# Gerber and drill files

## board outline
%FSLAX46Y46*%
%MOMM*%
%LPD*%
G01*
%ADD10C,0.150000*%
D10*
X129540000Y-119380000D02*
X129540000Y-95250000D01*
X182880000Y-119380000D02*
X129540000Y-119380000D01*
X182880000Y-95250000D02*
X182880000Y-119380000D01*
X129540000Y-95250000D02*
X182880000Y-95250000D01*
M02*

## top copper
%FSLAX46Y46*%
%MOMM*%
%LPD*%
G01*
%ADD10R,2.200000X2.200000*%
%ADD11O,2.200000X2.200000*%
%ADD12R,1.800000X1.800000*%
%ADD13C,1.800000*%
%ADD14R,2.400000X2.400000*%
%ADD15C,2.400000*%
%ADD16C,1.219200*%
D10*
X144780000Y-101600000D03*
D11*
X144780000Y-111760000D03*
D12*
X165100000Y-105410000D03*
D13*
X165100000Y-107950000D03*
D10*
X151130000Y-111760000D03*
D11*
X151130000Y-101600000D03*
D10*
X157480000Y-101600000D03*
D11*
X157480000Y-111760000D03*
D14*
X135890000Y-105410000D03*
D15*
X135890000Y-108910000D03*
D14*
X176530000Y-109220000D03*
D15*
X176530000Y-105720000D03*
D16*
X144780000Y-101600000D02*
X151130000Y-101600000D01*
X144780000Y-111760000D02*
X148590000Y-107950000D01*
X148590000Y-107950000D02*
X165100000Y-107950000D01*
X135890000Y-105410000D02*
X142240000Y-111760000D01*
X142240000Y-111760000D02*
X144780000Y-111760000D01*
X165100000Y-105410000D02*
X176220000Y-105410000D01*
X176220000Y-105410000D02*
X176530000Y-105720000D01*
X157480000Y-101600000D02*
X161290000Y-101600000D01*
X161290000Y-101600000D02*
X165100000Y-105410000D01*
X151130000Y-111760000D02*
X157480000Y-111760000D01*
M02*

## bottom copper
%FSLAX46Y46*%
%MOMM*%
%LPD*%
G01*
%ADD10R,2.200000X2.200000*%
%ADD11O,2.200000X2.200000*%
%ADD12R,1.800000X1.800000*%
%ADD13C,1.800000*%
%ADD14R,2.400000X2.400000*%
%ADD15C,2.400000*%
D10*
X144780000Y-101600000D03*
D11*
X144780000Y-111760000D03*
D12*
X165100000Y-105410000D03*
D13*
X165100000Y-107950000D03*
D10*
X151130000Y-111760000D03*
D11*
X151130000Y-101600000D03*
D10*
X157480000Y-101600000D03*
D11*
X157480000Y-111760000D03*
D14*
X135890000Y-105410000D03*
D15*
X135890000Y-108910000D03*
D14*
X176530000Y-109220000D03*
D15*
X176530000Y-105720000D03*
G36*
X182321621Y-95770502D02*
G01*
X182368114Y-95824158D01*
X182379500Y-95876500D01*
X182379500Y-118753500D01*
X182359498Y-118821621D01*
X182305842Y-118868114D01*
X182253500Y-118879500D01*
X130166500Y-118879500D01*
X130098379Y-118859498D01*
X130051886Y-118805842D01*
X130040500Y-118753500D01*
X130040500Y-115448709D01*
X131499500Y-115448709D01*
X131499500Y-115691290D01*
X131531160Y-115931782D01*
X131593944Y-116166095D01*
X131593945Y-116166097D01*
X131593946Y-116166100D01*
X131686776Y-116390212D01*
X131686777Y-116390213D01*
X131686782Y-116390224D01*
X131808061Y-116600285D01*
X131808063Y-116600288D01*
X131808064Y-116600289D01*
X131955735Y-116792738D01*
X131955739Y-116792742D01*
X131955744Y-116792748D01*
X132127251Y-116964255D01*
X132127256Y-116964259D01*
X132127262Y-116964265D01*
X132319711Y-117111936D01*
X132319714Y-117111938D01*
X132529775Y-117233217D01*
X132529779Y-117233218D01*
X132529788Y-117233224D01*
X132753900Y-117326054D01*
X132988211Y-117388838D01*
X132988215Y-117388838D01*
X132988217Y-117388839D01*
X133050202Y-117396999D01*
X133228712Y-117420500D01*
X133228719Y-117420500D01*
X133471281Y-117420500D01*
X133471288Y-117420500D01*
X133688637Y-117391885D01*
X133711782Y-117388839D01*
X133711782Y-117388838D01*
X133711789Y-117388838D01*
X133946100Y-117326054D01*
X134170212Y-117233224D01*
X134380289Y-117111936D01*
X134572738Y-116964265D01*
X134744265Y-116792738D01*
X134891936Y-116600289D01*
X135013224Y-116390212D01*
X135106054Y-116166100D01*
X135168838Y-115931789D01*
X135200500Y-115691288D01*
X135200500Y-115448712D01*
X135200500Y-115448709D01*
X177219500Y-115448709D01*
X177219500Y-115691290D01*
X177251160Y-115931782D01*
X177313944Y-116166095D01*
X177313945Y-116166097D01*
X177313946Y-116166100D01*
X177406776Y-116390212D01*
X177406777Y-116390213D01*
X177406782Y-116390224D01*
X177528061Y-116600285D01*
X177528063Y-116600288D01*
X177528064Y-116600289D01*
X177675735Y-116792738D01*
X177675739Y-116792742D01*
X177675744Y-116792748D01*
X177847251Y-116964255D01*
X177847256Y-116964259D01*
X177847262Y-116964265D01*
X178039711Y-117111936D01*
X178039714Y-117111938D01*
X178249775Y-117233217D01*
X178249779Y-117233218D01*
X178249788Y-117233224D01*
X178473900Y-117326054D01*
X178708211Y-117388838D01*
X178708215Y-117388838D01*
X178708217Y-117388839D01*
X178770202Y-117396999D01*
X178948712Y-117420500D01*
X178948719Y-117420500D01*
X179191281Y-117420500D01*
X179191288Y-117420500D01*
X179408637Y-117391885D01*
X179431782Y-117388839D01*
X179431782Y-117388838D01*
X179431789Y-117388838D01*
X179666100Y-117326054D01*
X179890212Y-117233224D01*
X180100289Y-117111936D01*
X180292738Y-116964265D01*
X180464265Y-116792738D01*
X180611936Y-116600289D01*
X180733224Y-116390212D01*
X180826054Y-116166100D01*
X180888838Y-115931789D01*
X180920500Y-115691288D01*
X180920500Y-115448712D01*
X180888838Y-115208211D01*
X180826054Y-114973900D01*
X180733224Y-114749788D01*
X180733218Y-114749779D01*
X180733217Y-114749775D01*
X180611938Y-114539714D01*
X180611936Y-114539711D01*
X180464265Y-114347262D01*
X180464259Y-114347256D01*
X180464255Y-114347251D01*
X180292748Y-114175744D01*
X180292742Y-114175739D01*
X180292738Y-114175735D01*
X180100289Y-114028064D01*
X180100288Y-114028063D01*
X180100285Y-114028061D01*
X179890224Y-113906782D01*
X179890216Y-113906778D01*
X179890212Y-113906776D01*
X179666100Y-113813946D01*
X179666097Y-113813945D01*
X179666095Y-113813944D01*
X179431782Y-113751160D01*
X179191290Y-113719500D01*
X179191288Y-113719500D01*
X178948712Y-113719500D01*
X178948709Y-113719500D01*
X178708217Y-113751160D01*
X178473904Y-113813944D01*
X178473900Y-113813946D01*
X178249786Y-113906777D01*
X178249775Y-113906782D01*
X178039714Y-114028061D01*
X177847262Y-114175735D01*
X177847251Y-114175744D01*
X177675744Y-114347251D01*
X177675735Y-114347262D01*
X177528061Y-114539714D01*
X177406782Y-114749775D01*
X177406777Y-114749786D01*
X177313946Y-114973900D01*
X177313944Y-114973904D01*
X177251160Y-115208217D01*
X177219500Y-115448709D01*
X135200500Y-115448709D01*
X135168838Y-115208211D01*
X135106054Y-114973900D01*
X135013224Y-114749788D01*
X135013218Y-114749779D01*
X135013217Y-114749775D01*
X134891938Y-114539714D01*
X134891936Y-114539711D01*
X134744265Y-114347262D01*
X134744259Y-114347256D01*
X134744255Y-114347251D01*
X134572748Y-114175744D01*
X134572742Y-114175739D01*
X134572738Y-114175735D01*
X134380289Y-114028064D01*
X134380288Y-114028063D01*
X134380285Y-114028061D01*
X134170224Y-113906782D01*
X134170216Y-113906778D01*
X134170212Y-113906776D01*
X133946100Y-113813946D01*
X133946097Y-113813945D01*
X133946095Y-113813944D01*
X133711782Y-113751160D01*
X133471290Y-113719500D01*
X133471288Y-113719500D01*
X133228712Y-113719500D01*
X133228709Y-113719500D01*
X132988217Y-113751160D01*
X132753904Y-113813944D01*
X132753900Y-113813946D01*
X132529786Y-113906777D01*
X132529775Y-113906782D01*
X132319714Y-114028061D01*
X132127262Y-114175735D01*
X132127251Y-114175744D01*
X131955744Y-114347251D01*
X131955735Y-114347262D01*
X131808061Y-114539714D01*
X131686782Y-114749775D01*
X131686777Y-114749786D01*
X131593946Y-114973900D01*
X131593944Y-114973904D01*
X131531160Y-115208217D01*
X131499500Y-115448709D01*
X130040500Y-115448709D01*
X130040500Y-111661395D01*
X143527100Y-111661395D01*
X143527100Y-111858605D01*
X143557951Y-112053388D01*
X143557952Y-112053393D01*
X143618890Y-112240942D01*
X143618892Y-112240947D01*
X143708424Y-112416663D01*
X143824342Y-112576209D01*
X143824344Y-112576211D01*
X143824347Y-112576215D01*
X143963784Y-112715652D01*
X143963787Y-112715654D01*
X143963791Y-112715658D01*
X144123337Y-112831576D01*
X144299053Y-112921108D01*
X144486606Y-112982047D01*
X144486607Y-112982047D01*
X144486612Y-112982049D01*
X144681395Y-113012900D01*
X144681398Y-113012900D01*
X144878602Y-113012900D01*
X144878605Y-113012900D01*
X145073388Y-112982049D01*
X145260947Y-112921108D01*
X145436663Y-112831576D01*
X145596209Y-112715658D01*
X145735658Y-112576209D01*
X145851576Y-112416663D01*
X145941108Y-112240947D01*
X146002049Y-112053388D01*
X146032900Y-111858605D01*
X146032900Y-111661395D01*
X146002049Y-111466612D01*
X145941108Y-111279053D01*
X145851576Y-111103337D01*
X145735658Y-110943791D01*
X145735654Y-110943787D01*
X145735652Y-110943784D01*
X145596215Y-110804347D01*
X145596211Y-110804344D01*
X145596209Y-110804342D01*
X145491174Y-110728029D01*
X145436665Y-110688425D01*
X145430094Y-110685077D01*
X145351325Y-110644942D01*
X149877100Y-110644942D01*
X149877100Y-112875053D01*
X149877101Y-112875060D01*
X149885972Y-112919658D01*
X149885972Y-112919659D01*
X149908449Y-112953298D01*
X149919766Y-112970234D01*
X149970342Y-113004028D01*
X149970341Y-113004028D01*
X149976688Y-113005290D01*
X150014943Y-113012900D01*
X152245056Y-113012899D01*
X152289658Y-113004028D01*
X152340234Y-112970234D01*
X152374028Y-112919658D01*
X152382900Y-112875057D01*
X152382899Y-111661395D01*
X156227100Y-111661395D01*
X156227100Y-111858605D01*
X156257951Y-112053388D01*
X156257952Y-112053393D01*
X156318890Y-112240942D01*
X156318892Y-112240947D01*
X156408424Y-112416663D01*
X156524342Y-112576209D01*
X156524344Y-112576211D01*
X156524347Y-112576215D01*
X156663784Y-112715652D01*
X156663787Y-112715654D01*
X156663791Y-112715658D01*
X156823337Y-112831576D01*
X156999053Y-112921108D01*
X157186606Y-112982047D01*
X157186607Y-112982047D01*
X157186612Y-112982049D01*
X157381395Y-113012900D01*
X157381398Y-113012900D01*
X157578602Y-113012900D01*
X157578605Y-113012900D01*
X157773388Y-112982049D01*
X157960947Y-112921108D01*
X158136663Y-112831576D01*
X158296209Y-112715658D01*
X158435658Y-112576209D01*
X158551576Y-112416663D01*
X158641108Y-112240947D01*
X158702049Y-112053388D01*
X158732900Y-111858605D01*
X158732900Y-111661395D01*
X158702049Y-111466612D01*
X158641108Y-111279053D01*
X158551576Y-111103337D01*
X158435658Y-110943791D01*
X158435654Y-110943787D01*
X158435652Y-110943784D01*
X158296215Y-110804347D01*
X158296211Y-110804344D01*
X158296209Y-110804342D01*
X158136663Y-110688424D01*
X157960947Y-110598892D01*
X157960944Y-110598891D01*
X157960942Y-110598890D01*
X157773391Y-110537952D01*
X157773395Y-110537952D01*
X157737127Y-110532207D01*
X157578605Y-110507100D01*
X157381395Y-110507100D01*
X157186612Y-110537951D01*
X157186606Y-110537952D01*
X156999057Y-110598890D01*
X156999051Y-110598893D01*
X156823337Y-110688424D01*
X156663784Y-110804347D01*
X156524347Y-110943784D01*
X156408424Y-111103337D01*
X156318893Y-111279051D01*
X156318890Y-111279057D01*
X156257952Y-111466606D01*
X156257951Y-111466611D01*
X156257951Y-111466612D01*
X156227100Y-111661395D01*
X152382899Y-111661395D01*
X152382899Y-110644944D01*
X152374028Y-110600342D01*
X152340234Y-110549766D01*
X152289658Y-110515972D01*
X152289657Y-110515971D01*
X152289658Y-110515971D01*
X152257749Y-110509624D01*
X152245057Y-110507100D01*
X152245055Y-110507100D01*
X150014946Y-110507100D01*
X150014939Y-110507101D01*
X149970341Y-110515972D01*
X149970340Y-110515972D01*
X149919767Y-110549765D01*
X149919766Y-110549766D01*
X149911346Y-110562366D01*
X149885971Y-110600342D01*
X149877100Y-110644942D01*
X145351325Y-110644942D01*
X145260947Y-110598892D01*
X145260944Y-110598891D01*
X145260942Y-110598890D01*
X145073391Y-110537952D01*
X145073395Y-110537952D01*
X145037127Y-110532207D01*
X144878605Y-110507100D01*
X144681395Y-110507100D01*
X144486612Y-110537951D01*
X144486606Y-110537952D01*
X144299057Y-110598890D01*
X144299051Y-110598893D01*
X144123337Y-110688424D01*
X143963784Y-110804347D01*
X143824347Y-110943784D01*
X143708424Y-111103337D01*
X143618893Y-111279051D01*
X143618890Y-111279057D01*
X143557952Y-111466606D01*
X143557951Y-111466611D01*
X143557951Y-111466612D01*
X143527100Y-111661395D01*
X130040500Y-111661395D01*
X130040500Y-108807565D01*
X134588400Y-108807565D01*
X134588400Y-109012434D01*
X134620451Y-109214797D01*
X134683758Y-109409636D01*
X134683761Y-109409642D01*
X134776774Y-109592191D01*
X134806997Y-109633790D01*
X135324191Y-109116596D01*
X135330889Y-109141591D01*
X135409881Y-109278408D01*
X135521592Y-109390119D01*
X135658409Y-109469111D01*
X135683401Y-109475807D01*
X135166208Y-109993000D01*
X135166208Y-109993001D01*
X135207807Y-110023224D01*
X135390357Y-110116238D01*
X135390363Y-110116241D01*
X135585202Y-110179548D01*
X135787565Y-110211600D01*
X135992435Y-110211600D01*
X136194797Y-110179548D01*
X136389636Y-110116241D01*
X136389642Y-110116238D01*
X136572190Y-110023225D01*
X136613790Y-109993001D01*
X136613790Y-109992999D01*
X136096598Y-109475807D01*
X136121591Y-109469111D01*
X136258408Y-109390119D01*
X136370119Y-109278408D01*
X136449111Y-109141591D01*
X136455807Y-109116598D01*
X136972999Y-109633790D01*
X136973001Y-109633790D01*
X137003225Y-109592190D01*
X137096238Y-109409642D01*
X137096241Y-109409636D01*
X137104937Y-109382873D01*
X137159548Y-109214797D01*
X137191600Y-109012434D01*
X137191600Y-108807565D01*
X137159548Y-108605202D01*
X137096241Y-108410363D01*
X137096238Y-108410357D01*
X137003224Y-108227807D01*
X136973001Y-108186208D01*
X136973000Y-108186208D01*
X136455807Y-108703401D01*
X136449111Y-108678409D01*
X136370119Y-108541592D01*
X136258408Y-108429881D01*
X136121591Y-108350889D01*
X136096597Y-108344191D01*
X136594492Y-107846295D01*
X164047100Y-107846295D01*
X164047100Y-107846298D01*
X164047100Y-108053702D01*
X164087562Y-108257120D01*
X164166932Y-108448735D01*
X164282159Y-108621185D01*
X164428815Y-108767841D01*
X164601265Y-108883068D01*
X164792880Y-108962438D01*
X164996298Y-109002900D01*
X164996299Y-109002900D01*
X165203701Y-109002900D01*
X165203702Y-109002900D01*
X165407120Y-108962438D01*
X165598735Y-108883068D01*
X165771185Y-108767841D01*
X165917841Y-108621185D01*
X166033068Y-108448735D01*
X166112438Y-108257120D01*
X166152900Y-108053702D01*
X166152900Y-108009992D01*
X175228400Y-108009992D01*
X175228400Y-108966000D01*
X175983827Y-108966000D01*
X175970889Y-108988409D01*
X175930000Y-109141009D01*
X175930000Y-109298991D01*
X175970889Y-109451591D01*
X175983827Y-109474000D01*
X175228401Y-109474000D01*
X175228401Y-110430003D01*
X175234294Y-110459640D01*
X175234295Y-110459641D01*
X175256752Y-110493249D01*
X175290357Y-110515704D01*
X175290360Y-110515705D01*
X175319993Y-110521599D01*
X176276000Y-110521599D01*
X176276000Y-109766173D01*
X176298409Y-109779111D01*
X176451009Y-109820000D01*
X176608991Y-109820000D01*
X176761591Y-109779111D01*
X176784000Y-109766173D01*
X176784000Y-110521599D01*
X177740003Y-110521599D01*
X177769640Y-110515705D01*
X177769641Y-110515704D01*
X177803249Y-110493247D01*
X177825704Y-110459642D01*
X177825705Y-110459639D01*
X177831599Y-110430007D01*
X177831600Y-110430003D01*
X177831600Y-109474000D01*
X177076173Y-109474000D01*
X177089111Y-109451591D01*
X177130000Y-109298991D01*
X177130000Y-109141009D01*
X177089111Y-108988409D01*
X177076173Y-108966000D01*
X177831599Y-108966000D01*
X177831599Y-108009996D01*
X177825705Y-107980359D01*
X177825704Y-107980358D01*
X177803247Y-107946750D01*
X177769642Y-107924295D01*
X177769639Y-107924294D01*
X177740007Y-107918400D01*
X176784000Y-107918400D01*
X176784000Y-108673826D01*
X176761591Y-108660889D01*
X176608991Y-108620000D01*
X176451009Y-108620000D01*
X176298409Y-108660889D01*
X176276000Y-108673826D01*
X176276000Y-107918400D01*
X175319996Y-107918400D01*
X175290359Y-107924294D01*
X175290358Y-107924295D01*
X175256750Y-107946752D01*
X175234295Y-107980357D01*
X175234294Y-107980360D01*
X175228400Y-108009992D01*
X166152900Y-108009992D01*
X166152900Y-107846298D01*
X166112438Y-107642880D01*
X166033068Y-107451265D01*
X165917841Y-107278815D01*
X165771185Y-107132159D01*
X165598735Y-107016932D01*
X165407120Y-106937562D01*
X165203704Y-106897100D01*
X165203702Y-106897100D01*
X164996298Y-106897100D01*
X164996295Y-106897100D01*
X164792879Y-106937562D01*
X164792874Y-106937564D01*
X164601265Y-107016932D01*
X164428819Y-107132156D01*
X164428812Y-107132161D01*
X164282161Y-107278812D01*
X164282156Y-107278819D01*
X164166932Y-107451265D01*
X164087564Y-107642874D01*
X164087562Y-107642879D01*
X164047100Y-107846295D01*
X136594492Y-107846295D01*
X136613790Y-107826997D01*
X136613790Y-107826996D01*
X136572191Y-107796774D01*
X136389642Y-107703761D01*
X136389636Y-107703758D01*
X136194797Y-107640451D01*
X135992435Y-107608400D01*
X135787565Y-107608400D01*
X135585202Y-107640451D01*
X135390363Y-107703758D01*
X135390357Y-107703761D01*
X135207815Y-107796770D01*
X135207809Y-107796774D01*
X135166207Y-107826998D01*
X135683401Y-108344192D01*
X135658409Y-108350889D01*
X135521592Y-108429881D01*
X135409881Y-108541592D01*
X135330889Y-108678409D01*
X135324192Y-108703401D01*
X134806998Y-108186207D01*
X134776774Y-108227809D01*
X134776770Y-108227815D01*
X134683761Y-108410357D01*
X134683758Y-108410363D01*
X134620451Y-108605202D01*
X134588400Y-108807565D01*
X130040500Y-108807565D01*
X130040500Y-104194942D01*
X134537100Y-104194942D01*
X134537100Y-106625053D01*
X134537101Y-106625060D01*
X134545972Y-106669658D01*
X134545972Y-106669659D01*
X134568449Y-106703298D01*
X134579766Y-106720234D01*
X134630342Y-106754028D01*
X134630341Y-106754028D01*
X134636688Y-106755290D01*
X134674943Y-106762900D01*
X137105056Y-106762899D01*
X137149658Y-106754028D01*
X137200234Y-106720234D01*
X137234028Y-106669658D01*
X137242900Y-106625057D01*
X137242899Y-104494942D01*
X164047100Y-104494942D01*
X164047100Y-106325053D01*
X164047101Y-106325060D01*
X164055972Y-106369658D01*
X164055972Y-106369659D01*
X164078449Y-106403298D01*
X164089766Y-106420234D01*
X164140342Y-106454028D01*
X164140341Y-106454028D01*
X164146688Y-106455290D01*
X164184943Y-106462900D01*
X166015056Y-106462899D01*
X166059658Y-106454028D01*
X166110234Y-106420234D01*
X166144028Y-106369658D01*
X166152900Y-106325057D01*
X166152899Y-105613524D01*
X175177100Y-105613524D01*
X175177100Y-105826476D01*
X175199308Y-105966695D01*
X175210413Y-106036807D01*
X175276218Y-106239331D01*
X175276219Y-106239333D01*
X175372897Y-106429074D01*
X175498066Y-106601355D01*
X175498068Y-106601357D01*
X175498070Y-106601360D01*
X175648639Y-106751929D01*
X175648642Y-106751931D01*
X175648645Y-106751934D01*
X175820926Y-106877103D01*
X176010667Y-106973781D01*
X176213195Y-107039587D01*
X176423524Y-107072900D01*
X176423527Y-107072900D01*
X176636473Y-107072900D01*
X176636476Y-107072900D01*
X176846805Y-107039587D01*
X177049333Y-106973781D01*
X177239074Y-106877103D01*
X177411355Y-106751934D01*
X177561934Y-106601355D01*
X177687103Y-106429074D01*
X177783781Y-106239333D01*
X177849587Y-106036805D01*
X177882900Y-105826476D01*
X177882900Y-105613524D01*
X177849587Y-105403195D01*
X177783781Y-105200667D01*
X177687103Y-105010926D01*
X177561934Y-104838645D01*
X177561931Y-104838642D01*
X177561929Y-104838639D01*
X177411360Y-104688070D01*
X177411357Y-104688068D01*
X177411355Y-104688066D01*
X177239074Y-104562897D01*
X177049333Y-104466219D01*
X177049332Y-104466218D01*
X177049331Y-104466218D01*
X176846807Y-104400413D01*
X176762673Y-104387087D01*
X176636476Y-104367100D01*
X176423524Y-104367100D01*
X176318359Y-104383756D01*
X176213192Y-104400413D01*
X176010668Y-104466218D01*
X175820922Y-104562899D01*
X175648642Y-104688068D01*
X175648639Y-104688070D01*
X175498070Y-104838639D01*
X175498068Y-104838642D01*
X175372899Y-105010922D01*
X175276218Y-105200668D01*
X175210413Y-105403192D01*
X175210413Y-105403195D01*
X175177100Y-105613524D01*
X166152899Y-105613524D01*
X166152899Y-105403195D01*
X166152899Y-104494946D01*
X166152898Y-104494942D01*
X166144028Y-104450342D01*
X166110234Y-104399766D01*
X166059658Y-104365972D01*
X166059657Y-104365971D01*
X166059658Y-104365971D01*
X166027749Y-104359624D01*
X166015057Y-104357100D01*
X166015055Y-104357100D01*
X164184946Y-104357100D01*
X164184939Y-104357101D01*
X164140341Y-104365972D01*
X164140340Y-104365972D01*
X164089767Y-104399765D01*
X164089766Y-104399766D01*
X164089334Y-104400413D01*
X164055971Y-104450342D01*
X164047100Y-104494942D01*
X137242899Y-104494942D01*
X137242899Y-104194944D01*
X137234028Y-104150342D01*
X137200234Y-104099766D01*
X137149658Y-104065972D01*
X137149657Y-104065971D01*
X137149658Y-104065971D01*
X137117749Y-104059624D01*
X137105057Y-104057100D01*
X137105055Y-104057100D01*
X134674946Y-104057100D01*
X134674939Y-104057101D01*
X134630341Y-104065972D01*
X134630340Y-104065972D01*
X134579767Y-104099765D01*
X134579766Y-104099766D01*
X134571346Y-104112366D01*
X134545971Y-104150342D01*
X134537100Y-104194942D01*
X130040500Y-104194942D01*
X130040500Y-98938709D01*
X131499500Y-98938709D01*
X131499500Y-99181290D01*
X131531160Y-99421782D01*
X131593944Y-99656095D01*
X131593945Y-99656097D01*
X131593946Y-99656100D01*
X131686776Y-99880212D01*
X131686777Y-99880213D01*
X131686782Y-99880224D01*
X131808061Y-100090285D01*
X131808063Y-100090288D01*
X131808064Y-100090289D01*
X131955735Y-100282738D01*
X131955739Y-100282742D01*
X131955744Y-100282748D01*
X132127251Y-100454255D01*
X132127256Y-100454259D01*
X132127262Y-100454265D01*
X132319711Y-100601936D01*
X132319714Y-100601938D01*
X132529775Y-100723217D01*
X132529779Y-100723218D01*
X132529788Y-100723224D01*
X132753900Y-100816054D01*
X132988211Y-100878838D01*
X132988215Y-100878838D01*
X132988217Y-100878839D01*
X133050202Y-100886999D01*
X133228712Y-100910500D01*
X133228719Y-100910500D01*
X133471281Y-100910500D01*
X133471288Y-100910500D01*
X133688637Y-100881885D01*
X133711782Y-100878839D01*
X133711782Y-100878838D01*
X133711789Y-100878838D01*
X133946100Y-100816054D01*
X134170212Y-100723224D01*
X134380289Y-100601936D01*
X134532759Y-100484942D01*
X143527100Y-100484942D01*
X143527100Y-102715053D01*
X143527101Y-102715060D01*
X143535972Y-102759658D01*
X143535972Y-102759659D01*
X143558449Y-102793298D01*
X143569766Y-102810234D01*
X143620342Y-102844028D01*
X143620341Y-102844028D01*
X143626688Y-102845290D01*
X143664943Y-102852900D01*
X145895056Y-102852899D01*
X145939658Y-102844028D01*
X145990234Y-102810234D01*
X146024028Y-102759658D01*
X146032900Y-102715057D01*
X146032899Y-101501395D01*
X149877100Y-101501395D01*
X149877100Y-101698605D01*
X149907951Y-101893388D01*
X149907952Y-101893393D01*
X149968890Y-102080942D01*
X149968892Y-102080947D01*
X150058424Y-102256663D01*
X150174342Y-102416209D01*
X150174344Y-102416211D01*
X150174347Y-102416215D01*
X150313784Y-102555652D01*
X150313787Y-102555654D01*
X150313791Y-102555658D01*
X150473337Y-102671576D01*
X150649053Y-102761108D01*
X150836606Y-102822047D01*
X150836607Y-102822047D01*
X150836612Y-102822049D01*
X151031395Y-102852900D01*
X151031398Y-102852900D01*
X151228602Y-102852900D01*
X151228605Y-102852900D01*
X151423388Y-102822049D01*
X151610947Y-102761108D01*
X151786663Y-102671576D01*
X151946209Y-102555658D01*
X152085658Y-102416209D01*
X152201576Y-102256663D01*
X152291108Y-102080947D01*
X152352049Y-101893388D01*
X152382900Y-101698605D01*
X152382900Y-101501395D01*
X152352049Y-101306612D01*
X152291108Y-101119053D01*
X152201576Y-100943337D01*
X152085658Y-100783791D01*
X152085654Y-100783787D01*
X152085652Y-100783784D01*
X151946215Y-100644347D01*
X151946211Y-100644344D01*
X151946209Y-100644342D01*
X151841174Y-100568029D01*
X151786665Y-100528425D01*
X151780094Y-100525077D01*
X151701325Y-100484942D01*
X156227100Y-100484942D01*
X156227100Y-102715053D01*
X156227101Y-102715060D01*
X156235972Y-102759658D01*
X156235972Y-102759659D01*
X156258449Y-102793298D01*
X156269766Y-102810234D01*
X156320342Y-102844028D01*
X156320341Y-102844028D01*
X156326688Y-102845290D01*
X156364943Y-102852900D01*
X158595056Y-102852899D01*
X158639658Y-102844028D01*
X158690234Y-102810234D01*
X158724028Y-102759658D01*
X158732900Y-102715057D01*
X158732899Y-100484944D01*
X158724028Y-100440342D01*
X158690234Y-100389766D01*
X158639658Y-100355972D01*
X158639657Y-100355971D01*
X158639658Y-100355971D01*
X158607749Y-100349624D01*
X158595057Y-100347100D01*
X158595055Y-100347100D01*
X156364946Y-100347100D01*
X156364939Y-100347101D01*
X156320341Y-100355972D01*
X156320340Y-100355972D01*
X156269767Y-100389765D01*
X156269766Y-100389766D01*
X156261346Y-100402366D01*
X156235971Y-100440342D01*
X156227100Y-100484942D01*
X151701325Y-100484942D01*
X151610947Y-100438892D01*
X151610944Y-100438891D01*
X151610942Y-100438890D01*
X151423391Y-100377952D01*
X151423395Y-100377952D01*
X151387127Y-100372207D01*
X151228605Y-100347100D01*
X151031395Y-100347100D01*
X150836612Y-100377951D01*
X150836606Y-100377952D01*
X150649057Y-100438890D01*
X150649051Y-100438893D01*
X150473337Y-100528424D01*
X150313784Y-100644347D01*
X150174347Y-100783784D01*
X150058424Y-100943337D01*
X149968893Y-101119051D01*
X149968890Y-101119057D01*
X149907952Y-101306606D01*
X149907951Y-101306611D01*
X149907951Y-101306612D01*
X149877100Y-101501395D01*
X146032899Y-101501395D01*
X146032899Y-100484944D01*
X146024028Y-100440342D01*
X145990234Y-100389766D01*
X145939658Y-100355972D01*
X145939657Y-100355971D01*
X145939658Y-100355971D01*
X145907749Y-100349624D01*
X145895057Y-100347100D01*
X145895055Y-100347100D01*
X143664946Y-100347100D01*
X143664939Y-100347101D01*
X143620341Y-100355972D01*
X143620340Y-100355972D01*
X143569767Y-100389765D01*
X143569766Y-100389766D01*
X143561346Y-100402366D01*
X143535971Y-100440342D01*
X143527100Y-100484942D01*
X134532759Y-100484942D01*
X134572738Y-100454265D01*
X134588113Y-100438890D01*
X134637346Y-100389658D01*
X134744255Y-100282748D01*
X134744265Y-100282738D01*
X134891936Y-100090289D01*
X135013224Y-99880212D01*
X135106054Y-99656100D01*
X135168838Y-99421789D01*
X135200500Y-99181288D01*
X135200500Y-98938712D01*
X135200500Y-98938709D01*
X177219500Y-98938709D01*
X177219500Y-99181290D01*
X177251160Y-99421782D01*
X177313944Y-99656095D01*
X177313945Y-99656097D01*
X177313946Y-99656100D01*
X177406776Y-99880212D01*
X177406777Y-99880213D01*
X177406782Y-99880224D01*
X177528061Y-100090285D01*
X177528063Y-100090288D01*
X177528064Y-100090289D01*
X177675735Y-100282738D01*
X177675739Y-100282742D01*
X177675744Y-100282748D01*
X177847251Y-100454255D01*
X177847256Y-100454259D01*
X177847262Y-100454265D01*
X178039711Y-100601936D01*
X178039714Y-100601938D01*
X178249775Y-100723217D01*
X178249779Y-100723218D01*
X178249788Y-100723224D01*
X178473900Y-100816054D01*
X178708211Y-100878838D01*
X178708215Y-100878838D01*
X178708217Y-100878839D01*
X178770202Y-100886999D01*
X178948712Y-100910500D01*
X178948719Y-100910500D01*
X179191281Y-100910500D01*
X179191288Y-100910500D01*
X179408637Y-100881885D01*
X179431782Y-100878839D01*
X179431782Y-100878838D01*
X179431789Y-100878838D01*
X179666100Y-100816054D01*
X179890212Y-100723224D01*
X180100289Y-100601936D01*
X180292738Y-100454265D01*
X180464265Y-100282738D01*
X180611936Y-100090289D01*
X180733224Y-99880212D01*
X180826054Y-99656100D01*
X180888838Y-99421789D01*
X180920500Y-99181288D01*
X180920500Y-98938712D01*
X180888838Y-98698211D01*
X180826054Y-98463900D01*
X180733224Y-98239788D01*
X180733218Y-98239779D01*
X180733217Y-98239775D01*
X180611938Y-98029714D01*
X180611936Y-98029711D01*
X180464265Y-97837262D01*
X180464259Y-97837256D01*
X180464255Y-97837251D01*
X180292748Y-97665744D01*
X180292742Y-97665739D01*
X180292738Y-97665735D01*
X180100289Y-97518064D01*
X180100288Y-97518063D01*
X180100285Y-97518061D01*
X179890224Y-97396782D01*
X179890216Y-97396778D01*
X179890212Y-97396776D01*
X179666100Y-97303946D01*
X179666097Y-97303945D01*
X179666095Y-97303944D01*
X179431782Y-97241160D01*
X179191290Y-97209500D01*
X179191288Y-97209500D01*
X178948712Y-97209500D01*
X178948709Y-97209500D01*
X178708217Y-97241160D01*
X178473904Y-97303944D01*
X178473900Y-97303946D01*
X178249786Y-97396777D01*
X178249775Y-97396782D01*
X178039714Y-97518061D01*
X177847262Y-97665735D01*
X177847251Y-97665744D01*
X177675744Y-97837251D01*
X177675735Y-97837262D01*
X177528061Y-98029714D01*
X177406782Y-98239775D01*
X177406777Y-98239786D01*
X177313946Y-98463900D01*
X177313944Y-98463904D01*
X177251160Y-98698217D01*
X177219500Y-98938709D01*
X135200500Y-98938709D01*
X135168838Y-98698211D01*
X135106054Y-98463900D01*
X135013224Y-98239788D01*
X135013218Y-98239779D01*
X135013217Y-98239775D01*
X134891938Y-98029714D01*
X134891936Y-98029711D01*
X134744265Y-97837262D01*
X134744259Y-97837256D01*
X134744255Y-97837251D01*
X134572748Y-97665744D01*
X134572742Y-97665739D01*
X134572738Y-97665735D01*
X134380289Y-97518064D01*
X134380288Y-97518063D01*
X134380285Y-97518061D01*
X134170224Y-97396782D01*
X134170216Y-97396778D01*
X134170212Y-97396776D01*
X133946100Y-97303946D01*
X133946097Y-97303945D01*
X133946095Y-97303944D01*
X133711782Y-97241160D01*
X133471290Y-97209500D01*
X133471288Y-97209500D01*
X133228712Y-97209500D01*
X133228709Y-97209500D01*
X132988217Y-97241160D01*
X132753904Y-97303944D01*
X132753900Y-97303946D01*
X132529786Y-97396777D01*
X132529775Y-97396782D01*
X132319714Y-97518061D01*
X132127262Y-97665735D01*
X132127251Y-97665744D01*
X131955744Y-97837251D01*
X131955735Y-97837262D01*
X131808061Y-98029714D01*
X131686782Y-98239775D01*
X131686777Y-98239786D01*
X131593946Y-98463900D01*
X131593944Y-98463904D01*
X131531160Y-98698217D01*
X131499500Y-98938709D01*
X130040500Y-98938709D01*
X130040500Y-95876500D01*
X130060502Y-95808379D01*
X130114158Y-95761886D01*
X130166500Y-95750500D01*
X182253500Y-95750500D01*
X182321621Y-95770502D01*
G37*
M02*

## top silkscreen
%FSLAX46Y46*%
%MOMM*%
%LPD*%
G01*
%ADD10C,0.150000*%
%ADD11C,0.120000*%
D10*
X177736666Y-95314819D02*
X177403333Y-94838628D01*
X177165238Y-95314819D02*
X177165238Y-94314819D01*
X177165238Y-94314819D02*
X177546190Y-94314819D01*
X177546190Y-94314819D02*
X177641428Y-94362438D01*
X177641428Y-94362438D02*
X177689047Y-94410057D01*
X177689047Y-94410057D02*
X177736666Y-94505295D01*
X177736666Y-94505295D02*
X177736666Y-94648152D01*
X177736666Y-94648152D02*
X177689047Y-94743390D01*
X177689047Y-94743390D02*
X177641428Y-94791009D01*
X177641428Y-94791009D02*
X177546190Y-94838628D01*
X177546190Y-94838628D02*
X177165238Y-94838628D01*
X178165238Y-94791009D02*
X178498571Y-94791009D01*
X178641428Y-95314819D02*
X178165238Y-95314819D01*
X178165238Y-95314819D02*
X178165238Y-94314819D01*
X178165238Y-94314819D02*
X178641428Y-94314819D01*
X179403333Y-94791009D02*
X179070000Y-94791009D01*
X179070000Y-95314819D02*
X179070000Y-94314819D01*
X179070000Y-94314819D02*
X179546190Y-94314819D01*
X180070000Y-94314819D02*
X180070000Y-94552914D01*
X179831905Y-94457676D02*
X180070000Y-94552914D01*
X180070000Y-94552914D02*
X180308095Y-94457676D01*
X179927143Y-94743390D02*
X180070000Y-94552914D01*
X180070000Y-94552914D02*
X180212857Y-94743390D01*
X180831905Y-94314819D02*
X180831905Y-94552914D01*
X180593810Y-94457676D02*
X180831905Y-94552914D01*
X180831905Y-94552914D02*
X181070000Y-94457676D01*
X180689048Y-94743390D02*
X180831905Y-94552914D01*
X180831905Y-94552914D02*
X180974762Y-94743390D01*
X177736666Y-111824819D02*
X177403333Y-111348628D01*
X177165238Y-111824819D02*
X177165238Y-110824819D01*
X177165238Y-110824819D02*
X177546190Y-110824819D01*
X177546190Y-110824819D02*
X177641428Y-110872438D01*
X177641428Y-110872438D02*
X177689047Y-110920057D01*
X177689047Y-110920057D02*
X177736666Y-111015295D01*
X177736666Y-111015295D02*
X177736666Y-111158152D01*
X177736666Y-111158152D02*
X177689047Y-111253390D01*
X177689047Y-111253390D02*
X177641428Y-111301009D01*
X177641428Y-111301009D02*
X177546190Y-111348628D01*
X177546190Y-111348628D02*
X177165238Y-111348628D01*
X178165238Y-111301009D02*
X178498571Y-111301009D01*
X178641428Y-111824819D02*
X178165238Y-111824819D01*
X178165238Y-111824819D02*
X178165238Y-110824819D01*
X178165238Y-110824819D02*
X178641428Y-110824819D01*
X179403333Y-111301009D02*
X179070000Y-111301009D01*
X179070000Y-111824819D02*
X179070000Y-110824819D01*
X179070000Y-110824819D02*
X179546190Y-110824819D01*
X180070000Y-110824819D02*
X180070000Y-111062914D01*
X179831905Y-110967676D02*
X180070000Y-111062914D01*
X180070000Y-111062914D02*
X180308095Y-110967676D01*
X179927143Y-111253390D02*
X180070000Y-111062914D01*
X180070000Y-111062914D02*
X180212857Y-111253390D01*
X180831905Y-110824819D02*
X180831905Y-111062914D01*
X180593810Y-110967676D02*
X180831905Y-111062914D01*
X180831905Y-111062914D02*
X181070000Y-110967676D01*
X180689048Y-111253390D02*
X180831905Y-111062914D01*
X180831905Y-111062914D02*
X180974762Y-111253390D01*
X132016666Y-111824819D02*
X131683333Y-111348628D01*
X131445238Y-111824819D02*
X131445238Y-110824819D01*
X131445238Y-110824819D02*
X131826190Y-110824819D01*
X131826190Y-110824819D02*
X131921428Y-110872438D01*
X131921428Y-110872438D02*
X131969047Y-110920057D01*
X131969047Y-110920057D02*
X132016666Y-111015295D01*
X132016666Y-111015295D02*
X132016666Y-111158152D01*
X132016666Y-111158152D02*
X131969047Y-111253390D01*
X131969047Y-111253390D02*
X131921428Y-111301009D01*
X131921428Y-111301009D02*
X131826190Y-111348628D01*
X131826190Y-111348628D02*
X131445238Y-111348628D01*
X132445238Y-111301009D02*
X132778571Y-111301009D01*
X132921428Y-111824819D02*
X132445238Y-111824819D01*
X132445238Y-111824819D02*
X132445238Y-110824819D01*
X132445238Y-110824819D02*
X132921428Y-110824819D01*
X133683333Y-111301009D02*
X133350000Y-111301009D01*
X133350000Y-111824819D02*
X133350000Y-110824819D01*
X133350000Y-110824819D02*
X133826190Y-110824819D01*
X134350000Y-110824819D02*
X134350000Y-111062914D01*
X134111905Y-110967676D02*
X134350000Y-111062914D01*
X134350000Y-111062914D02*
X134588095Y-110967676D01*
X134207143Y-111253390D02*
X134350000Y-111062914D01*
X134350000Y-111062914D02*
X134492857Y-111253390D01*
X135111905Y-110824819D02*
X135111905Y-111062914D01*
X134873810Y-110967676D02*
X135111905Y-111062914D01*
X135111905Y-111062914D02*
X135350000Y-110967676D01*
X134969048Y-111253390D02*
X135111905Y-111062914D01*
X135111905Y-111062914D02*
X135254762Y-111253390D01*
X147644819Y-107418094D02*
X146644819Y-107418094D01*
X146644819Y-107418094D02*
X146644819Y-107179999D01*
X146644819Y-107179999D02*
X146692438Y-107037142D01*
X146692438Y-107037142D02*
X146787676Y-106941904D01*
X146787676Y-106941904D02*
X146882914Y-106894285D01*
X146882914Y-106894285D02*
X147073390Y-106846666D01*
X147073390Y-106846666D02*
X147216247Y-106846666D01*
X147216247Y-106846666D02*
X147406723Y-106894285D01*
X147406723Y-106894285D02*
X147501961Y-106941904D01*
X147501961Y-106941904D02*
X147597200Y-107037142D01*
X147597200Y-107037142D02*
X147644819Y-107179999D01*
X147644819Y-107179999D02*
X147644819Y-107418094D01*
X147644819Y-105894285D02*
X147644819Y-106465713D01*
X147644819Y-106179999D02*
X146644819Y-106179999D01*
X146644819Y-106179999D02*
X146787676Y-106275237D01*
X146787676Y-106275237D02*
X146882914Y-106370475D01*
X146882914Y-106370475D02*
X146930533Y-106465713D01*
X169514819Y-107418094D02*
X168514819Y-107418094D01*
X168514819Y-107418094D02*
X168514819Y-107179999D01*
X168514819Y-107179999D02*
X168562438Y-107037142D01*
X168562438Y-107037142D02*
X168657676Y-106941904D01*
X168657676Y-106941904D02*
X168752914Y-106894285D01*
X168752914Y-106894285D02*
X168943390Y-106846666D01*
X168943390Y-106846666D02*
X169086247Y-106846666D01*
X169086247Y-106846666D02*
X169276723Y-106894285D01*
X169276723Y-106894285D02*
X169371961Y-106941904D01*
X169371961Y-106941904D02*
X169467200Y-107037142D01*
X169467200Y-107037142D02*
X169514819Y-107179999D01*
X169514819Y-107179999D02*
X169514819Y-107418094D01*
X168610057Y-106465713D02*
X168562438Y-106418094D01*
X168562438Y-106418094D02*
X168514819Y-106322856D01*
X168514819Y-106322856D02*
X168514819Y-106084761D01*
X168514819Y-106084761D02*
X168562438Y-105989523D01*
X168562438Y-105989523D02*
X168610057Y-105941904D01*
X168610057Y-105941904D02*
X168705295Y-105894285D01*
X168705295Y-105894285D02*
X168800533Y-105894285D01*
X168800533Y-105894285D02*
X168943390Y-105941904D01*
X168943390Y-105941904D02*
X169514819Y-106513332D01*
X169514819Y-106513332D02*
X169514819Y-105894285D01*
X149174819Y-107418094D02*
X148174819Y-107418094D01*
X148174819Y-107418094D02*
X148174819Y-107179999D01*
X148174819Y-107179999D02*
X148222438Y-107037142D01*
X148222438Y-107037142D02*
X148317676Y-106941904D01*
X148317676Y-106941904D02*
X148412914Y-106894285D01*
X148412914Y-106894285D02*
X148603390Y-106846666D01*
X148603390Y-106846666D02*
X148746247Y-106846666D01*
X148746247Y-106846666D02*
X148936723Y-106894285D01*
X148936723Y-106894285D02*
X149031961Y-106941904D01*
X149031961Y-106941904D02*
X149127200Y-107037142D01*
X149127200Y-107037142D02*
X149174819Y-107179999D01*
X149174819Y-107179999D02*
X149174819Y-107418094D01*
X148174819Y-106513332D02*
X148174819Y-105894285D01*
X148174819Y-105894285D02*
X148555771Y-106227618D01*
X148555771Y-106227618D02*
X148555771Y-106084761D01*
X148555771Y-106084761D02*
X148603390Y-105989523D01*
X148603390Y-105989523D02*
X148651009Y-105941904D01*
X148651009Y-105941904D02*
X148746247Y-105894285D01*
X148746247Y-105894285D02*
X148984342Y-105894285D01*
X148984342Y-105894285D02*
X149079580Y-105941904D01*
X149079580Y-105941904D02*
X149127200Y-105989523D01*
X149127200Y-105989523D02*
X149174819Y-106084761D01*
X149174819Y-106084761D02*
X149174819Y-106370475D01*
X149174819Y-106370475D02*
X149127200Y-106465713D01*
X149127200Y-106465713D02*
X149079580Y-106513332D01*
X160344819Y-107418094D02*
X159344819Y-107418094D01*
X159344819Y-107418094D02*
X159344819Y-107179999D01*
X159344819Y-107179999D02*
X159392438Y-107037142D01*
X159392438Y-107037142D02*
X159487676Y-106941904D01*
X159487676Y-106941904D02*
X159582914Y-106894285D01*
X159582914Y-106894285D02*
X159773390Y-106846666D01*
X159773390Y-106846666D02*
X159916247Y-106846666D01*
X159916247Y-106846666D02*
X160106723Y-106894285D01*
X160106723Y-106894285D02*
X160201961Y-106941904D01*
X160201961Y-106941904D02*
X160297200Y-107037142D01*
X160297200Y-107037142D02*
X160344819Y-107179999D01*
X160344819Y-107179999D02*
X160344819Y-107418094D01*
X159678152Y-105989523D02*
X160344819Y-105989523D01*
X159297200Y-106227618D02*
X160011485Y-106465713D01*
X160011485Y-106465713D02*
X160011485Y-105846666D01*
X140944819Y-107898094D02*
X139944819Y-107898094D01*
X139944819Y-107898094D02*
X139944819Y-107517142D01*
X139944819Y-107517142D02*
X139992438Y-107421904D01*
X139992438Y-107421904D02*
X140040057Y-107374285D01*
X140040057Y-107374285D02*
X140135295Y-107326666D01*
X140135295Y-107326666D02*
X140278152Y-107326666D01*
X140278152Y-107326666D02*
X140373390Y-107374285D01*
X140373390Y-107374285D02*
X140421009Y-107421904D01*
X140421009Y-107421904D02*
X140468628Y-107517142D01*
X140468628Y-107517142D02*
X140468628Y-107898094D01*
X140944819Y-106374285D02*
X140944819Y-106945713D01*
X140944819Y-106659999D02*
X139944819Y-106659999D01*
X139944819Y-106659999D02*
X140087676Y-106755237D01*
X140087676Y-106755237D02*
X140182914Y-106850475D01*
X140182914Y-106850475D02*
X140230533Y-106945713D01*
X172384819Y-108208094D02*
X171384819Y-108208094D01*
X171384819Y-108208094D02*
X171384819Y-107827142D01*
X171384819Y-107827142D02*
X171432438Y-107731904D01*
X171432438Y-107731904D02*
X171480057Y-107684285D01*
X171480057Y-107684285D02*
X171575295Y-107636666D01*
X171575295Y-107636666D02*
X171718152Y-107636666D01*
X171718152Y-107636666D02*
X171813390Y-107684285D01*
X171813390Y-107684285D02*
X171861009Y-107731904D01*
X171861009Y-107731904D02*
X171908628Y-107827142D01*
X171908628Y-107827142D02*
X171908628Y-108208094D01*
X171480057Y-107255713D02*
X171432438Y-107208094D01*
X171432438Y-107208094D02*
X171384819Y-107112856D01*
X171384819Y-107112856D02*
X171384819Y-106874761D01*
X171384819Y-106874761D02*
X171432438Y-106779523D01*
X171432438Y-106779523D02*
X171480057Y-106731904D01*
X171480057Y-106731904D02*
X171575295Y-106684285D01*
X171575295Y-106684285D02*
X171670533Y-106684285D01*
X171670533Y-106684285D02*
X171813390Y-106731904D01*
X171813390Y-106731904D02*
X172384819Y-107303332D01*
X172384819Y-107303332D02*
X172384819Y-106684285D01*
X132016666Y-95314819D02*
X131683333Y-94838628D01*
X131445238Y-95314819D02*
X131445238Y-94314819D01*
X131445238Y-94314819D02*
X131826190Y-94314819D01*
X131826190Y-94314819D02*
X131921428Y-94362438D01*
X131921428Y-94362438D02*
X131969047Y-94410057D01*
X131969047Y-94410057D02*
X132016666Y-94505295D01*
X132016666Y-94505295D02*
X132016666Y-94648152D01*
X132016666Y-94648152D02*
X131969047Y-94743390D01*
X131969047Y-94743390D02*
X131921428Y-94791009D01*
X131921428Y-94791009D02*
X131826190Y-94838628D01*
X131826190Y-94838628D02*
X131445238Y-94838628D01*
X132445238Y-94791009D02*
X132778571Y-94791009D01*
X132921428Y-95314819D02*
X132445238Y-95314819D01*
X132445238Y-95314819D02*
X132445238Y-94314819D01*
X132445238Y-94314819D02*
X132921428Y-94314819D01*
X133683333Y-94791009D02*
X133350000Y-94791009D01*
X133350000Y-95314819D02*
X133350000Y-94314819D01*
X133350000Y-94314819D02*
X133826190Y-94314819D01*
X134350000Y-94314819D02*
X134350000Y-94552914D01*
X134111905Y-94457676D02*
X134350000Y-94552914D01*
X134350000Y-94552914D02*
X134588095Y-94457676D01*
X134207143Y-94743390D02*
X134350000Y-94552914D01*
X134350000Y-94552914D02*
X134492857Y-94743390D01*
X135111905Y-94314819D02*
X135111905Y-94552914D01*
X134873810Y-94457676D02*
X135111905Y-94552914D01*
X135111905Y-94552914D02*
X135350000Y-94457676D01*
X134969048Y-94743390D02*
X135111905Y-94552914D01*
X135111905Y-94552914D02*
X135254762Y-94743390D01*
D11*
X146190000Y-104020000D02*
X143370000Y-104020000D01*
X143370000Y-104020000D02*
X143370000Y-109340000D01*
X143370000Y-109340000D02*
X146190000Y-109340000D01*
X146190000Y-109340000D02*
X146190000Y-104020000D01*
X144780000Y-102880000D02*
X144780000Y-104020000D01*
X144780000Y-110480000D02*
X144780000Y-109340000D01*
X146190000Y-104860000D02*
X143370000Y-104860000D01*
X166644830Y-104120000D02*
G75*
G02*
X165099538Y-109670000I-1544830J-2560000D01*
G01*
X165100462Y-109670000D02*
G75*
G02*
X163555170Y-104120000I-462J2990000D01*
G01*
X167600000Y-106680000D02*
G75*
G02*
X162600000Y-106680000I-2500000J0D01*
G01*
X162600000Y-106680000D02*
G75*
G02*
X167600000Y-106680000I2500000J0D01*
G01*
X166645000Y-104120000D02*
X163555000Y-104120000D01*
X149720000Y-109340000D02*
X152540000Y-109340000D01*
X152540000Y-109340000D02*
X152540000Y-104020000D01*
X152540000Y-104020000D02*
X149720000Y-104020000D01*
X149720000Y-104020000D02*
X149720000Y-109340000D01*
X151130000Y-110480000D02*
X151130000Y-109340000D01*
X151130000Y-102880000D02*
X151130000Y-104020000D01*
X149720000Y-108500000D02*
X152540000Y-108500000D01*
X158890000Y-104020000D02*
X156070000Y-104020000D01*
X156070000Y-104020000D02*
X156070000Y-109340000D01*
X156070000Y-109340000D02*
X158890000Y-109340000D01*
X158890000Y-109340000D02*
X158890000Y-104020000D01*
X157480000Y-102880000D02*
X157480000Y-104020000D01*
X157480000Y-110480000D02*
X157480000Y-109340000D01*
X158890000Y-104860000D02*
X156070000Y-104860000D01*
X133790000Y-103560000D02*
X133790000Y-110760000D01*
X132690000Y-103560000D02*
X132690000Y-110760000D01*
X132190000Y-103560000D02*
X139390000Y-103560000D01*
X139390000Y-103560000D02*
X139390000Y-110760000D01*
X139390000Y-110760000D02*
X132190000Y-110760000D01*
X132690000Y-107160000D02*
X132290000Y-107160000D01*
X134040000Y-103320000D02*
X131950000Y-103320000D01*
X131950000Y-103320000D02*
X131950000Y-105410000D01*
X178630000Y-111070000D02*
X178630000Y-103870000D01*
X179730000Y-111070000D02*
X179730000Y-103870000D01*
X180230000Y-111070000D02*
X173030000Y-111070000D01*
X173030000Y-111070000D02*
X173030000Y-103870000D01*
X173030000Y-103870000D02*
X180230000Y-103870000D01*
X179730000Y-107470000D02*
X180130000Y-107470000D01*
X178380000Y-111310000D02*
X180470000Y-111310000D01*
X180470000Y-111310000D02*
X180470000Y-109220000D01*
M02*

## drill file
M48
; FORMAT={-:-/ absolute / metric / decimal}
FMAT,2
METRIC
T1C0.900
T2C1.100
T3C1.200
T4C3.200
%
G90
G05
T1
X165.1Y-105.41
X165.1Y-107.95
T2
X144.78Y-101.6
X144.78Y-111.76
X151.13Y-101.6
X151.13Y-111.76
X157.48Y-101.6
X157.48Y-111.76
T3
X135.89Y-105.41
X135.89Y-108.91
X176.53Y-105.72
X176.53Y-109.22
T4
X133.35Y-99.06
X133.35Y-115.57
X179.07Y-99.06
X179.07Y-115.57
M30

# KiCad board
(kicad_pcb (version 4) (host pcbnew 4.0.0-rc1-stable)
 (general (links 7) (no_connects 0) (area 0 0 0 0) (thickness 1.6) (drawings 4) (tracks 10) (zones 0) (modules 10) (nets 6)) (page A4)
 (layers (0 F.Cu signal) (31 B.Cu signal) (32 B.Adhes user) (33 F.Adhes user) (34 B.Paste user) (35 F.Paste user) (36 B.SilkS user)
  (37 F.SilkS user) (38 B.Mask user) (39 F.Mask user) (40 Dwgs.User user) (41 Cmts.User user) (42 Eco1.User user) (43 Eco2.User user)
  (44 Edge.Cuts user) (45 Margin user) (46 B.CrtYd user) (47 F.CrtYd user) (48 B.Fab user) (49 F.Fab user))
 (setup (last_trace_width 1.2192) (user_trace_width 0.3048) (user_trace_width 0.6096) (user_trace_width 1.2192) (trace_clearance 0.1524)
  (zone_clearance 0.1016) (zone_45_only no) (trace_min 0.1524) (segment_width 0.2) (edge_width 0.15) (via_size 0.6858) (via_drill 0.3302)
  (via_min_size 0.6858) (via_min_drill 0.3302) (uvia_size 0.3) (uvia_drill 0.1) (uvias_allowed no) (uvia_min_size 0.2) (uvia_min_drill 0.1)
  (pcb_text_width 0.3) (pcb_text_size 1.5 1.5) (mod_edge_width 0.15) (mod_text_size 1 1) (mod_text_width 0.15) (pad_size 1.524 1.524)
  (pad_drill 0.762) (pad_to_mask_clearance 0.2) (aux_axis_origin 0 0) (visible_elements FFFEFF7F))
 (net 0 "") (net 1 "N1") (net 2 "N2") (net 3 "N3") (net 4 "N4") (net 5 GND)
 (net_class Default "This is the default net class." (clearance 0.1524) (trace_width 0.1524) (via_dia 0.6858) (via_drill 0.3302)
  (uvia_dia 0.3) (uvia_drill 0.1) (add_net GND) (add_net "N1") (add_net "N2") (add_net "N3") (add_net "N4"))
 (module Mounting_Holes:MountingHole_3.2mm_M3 (layer F.Cu) (at 179.07 99.06)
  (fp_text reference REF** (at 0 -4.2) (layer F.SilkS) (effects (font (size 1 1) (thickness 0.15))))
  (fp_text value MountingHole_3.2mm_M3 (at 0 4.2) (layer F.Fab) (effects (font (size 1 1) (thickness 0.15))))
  (pad 1 np_thru_hole circle (at 0 0) (size 3.2 3.2) (drill 3.2) (layers *.Cu *.Mask)))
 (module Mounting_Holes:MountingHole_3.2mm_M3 (layer F.Cu) (at 179.07 115.57)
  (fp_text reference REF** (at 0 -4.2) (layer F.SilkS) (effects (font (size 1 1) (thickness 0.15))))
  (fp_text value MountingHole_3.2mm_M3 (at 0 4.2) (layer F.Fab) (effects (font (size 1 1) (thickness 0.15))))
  (pad 1 np_thru_hole circle (at 0 0) (size 3.2 3.2) (drill 3.2) (layers *.Cu *.Mask)))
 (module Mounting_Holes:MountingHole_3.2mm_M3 (layer F.Cu) (at 133.35 115.57)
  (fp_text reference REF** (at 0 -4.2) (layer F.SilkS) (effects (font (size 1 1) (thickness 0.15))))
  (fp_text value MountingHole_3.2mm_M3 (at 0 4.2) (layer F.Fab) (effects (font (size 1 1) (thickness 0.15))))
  (pad 1 np_thru_hole circle (at 0 0) (size 3.2 3.2) (drill 3.2) (layers *.Cu *.Mask)))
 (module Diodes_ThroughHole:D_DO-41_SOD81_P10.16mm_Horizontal (layer F.Cu) (at 144.78 101.6 270)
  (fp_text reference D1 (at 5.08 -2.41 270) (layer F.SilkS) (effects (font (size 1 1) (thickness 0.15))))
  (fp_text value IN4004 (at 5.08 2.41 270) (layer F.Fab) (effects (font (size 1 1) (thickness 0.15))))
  (fp_line (start 2.42 -1.41) (end 2.42 1.41) (layer F.SilkS) (width 0.12))
  (fp_line (start 2.42 1.41) (end 7.74 1.41) (layer F.SilkS) (width 0.12))
  (fp_line (start 7.74 1.41) (end 7.74 -1.41) (layer F.SilkS) (width 0.12))
  (fp_line (start 7.74 -1.41) (end 2.42 -1.41) (layer F.SilkS) (width 0.12))
  (fp_line (start 1.28 0) (end 2.42 0) (layer F.SilkS) (width 0.12))
  (fp_line (start 8.88 0) (end 7.74 0) (layer F.SilkS) (width 0.12))
  (fp_line (start 3.26 -1.41) (end 3.26 1.41) (layer F.SilkS) (width 0.12))
  (pad 1 thru_hole rect (at 0 0 270) (size 2.2 2.2) (drill 1.1) (layers *.Cu *.Mask) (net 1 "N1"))
  (pad 2 thru_hole oval (at 10.16 0 270) (size 2.2 2.2) (drill 1.1) (layers *.Cu *.Mask) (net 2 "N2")))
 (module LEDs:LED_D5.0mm (layer F.Cu) (at 165.1 105.41 270)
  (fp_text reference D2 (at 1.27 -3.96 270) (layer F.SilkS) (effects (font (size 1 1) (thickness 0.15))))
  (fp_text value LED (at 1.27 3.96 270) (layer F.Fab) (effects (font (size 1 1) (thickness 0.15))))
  (fp_arc (start 1.27 0) (end -1.29 -1.54483) (angle 148.9) (layer F.SilkS) (width 0.12))
  (fp_arc (start 1.27 0) (end -1.29 1.54483) (angle -148.9) (layer F.SilkS) (width 0.12))
  (fp_circle (center 1.27 0) (end 3.77 0) (layer F.SilkS) (width 0.12))
  (fp_line (start -1.29 -1.545) (end -1.29 1.545) (layer F.SilkS) (width 0.12))
  (pad 1 thru_hole rect (at 0 0 270) (size 1.8 1.8) (drill 0.9) (layers *.Cu *.Mask) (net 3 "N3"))
  (pad 2 thru_hole circle (at 2.54 0 270) (size 1.8 1.8) (drill 0.9) (layers *.Cu *.Mask) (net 2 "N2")))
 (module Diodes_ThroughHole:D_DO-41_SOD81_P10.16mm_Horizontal (layer F.Cu) (at 151.13 111.76 90)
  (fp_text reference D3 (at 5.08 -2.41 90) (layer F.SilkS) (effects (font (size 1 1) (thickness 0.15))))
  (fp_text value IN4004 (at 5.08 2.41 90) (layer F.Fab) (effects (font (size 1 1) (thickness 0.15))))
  (fp_line (start 2.42 -1.41) (end 2.42 1.41) (layer F.SilkS) (width 0.12))
  (fp_line (start 2.42 1.41) (end 7.74 1.41) (layer F.SilkS) (width 0.12))
  (fp_line (start 7.74 1.41) (end 7.74 -1.41) (layer F.SilkS) (width 0.12))
  (fp_line (start 7.74 -1.41) (end 2.42 -1.41) (layer F.SilkS) (width 0.12))
  (fp_line (start 1.28 0) (end 2.42 0) (layer F.SilkS) (width 0.12))
  (fp_line (start 8.88 0) (end 7.74 0) (layer F.SilkS) (width 0.12))
  (fp_line (start 3.26 -1.41) (end 3.26 1.41) (layer F.SilkS) (width 0.12))
  (pad 1 thru_hole rect (at 0 0 90) (size 2.2 2.2) (drill 1.1) (layers *.Cu *.Mask) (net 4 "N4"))
  (pad 2 thru_hole oval (at 10.16 0 90) (size 2.2 2.2) (drill 1.1) (layers *.Cu *.Mask) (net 1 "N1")))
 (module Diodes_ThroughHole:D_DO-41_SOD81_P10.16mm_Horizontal (layer F.Cu) (at 157.48 101.6 270)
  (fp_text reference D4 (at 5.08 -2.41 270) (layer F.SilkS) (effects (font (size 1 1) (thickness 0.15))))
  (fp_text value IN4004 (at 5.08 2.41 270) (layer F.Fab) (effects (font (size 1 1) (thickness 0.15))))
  (fp_line (start 2.42 -1.41) (end 2.42 1.41) (layer F.SilkS) (width 0.12))
  (fp_line (start 2.42 1.41) (end 7.74 1.41) (layer F.SilkS) (width 0.12))
  (fp_line (start 7.74 1.41) (end 7.74 -1.41) (layer F.SilkS) (width 0.12))
  (fp_line (start 7.74 -1.41) (end 2.42 -1.41) (layer F.SilkS) (width 0.12))
  (fp_line (start 1.28 0) (end 2.42 0) (layer F.SilkS) (width 0.12))
  (fp_line (start 8.88 0) (end 7.74 0) (layer F.SilkS) (width 0.12))
  (fp_line (start 3.26 -1.41) (end 3.26 1.41) (layer F.SilkS) (width 0.12))
  (pad 1 thru_hole rect (at 0 0 270) (size 2.2 2.2) (drill 1.1) (layers *.Cu *.Mask) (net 3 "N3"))
  (pad 2 thru_hole oval (at 10.16 0 270) (size 2.2 2.2) (drill 1.1) (layers *.Cu *.Mask) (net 4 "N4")))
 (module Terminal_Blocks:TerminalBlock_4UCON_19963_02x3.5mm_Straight (layer F.Cu) (at 135.89 105.41 270)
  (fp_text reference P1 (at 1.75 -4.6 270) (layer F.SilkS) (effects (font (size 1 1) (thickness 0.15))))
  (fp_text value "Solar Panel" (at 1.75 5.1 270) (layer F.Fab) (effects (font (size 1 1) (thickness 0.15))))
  (fp_line (start -1.85 2.1) (end 5.35 2.1) (layer F.SilkS) (width 0.12))
  (fp_line (start -1.85 3.2) (end 5.35 3.2) (layer F.SilkS) (width 0.12))
  (fp_line (start -1.85 3.7) (end -1.85 -3.5) (layer F.SilkS) (width 0.12))
  (fp_line (start -1.85 -3.5) (end 5.35 -3.5) (layer F.SilkS) (width 0.12))
  (fp_line (start 5.35 -3.5) (end 5.35 3.7) (layer F.SilkS) (width 0.12))
  (fp_line (start 1.75 3.2) (end 1.75 3.6) (layer F.SilkS) (width 0.12))
  (fp_line (start -2.09 1.85) (end -2.09 3.94) (layer F.SilkS) (width 0.12))
  (fp_line (start -2.09 3.94) (end 0 3.94) (layer F.SilkS) (width 0.12))
  (pad 1 thru_hole rect (at 0 0 270) (size 2.4 2.4) (drill 1.2) (layers *.Cu *.Mask) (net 2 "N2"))
  (pad 2 thru_hole circle (at 3.5 0 270) (size 2.4 2.4) (drill 1.2) (layers *.Cu *.Mask) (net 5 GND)))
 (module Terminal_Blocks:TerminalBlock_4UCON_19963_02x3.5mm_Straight (layer F.Cu) (at 176.53 109.22 90)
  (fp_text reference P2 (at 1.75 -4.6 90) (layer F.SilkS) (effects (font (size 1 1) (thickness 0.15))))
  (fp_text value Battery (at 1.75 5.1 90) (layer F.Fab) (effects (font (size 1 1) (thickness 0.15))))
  (fp_line (start -1.85 2.1) (end 5.35 2.1) (layer F.SilkS) (width 0.12))
  (fp_line (start -1.85 3.2) (end 5.35 3.2) (layer F.SilkS) (width 0.12))
  (fp_line (start -1.85 3.7) (end -1.85 -3.5) (layer F.SilkS) (width 0.12))
  (fp_line (start -1.85 -3.5) (end 5.35 -3.5) (layer F.SilkS) (width 0.12))
  (fp_line (start 5.35 -3.5) (end 5.35 3.7) (layer F.SilkS) (width 0.12))
  (fp_line (start 1.75 3.2) (end 1.75 3.6) (layer F.SilkS) (width 0.12))
  (fp_line (start -2.09 1.85) (end -2.09 3.94) (layer F.SilkS) (width 0.12))
  (fp_line (start -2.09 3.94) (end 0 3.94) (layer F.SilkS) (width 0.12))
  (pad 1 thru_hole rect (at 0 0 90) (size 2.4 2.4) (drill 1.2) (layers *.Cu *.Mask) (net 5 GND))
  (pad 2 thru_hole circle (at 3.5 0 90) (size 2.4 2.4) (drill 1.2) (layers *.Cu *.Mask) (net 3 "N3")))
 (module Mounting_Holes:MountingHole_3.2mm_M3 (layer F.Cu) (at 133.35 99.06)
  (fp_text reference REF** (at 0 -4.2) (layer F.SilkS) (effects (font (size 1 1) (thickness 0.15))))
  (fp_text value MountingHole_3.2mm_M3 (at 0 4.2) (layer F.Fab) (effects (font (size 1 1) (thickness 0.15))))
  (pad 1 np_thru_hole circle (at 0 0) (size 3.2 3.2) (drill 3.2) (layers *.Cu *.Mask)))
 (gr_line (start 129.54 119.38) (end 129.54 95.25) (angle 90) (layer Edge.Cuts) (width 0.15))
 (gr_line (start 182.88 119.38) (end 129.54 119.38) (angle 90) (layer Edge.Cuts) (width 0.15))
 (gr_line (start 182.88 95.25) (end 182.88 119.38) (angle 90) (layer Edge.Cuts) (width 0.15))
 (gr_line (start 129.54 95.25) (end 182.88 95.25) (angle 90) (layer Edge.Cuts) (width 0.15))
 (segment (start 144.78 101.6) (end 151.13 101.6) (width 1.2192) (layer F.Cu) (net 1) (status C00000))
 (segment (start 144.78 111.76) (end 148.59 107.95) (width 1.2192) (layer F.Cu) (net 2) (status 400000))
 (segment (start 148.59 107.95) (end 165.1 107.95) (width 1.2192) (layer F.Cu) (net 2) (status 800000))
 (segment (start 135.89 105.41) (end 142.24 111.76) (width 1.2192) (layer F.Cu) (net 2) (status 400000))
 (segment (start 142.24 111.76) (end 144.78 111.76) (width 1.2192) (layer F.Cu) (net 2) (status 800000))
 (segment (start 165.1 105.41) (end 176.22 105.41) (width 1.2192) (layer F.Cu) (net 3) (status C00000))
 (segment (start 176.22 105.41) (end 176.53 105.72) (width 1.2192) (layer F.Cu) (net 3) (status C00000))
 (segment (start 157.48 101.6) (end 161.29 101.6) (width 1.2192) (layer F.Cu) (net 3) (status 400000))
 (segment (start 161.29 101.6) (end 165.1 105.41) (width 1.2192) (layer F.Cu) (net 3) (status 800000))
 (segment (start 151.13 111.76) (end 157.48 111.76) (width 1.2192) (layer F.Cu) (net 4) (status C00000))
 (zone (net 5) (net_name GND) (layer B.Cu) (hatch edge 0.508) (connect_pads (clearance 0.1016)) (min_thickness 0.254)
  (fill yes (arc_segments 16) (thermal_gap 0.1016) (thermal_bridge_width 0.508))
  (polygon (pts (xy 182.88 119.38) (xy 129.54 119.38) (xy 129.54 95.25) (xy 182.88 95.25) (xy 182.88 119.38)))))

